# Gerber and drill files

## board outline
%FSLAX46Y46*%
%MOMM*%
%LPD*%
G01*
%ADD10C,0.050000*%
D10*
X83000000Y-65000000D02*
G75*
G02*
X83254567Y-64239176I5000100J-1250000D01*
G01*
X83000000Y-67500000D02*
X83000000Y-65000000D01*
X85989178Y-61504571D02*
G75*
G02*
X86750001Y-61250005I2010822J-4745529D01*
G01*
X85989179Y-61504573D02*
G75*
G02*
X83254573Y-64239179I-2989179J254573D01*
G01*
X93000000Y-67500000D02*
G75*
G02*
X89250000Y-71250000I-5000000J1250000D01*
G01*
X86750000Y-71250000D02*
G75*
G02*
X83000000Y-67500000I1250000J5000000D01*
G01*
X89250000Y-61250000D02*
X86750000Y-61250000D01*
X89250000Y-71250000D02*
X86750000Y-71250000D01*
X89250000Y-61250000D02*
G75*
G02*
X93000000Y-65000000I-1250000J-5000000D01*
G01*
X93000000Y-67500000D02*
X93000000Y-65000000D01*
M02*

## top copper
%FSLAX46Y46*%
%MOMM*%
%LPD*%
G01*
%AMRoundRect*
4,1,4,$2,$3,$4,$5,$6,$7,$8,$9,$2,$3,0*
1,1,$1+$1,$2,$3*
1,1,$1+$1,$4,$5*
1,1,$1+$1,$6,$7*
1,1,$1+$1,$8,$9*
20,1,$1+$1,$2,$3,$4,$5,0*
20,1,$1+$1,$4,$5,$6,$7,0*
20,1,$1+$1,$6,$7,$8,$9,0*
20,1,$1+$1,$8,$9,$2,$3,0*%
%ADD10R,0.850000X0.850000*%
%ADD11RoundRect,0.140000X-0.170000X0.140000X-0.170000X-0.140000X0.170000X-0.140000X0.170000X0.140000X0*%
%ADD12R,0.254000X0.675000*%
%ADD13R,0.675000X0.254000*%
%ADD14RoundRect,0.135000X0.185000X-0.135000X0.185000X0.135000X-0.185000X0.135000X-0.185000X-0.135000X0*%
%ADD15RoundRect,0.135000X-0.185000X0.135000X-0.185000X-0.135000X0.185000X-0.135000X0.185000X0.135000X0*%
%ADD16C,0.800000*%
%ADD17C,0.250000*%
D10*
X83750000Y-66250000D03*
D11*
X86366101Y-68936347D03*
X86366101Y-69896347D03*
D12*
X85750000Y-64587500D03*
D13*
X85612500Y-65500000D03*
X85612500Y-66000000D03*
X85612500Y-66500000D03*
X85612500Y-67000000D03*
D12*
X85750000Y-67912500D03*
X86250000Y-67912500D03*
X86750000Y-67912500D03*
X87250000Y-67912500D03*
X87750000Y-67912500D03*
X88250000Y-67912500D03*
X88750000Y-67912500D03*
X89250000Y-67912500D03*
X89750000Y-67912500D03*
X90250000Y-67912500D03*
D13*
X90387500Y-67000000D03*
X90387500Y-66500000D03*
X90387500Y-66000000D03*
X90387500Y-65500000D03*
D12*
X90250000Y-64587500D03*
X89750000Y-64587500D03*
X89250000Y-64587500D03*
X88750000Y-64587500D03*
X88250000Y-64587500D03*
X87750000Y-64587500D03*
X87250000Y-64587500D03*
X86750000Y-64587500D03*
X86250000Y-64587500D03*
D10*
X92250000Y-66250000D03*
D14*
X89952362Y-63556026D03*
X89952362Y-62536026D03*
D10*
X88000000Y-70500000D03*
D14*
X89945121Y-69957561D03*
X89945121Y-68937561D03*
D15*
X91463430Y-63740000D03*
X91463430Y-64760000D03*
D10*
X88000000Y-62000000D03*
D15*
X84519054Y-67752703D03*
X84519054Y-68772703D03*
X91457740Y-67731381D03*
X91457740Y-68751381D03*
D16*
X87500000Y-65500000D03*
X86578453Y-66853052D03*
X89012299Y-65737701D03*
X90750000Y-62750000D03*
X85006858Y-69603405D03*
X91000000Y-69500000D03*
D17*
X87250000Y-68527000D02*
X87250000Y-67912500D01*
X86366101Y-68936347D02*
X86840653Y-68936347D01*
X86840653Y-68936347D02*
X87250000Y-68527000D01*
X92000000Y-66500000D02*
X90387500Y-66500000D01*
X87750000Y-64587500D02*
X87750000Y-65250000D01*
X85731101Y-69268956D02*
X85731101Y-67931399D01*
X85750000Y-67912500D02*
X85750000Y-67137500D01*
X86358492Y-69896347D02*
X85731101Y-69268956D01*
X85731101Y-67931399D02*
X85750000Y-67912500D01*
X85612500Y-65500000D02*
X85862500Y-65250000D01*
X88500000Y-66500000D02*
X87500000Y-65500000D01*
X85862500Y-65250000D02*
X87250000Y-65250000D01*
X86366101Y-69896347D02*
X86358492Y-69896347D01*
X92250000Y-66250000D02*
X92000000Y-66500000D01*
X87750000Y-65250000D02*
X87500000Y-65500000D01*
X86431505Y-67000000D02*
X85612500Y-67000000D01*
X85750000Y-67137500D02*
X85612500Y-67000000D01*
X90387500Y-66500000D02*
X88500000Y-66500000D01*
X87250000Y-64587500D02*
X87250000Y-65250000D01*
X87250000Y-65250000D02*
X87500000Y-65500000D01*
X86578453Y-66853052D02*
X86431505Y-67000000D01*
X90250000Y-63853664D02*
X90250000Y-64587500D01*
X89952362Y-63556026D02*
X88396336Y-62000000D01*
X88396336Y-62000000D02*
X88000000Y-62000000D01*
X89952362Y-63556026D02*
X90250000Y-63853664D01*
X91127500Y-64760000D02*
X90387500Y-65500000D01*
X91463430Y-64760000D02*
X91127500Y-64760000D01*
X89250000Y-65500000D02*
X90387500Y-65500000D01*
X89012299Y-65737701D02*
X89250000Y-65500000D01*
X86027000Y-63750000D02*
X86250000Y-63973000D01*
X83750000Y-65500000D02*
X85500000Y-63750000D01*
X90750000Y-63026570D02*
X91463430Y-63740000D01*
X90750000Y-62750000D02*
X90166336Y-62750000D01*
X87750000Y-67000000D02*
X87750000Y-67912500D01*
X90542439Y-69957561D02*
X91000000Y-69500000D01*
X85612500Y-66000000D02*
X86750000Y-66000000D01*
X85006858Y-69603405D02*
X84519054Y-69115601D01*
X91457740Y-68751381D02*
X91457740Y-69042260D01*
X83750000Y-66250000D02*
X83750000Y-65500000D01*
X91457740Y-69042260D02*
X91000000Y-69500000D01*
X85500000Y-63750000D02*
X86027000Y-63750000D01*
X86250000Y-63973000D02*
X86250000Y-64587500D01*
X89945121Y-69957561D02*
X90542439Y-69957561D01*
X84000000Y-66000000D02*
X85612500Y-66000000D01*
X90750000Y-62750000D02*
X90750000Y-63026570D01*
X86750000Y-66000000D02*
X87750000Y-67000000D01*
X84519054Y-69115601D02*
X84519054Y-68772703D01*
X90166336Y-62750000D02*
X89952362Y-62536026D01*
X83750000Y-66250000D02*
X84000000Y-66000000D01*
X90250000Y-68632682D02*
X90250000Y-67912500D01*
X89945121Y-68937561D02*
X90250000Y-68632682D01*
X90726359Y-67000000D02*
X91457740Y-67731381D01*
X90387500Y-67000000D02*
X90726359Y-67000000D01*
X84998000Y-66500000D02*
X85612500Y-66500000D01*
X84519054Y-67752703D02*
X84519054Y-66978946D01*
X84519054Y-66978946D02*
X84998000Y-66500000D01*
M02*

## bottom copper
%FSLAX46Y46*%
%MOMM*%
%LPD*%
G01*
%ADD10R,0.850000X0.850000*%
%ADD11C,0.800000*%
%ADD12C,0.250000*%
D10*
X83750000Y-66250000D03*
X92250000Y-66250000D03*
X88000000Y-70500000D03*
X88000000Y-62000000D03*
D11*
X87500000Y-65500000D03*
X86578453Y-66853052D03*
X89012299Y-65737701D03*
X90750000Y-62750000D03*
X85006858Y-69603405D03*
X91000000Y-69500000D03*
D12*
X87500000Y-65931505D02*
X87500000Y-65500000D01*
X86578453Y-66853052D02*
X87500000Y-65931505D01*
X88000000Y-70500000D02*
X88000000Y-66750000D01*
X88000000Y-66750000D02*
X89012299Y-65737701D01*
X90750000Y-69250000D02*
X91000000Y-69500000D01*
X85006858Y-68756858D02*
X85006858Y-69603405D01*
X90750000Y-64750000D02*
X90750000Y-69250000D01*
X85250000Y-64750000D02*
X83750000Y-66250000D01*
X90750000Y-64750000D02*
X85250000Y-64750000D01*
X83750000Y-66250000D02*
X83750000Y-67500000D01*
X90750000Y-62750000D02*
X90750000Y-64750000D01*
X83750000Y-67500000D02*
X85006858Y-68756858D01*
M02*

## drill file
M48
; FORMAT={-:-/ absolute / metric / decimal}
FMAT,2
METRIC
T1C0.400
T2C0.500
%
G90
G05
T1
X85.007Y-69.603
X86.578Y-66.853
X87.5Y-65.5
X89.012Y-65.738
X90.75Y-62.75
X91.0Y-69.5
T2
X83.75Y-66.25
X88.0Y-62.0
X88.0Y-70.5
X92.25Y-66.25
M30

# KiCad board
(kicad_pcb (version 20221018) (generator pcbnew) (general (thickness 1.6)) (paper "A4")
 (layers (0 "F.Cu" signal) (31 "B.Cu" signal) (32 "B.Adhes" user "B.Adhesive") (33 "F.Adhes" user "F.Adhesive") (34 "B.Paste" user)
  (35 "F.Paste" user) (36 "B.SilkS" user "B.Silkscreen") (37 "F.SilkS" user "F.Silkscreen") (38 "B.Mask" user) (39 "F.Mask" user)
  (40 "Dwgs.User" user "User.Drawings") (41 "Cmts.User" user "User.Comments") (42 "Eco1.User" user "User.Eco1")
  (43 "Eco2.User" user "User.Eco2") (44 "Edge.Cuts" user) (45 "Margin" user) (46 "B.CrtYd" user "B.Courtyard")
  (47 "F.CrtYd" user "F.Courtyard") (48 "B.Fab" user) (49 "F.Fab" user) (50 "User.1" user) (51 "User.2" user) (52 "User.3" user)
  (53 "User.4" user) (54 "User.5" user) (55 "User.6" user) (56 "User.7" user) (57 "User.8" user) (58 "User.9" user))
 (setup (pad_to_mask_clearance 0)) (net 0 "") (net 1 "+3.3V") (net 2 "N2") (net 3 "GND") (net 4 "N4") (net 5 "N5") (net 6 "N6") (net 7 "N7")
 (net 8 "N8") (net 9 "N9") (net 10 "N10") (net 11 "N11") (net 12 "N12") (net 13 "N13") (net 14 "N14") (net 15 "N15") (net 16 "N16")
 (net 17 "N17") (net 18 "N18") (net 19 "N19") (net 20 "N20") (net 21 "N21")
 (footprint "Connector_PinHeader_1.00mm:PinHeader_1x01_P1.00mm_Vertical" (layer "F.Cu") (at 83.75 66.25)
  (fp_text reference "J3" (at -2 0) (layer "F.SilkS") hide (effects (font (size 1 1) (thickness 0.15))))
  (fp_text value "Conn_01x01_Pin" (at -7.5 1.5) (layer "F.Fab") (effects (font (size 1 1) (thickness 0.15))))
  (pad "1" thru_hole rect (at 0 0) (size 0.85 0.85) (drill 0.5) (layers "*.Cu" "*.Mask") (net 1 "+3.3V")))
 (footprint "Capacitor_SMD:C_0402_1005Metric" (layer "F.Cu") (at 86.366101 69.416347 -90)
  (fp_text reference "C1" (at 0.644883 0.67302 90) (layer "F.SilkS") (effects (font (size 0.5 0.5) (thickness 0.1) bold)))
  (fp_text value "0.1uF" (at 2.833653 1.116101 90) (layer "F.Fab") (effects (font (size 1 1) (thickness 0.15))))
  (pad "1" smd roundrect (at -0.48 0 270) (size 0.56 0.62) (layers "F.Cu" "F.Paste" "F.Mask") (roundrect_rratio 0.25) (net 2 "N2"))
  (pad "2" smd roundrect (at 0.48 0 270) (size 0.56 0.62) (layers "F.Cu" "F.Paste" "F.Mask") (roundrect_rratio 0.25) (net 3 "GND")))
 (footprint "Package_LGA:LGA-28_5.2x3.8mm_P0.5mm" (layer "F.Cu") (at 88 66.25)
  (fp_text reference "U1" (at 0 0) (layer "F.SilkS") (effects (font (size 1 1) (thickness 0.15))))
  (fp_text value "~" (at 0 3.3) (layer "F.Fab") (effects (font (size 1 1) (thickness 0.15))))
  (pad "1" smd rect (at -2.25 -1.6625) (size 0.254 0.675) (layers "F.Cu" "F.Paste" "F.Mask") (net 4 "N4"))
  (pad "2" smd rect (at -2.3875 -0.75 90) (size 0.254 0.675) (layers "F.Cu" "F.Paste" "F.Mask") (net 3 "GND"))
  (pad "3" smd rect (at -2.3875 -0.25 90) (size 0.254 0.675) (layers "F.Cu" "F.Paste" "F.Mask") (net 1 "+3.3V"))
  (pad "4" smd rect (at -2.3875 0.25 90) (size 0.254 0.675) (layers "F.Cu" "F.Paste" "F.Mask") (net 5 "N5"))
  (pad "5" smd rect (at -2.3875 0.75 90) (size 0.254 0.675) (layers "F.Cu" "F.Paste" "F.Mask") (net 3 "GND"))
  (pad "6" smd rect (at -2.25 1.6625) (size 0.254 0.675) (layers "F.Cu" "F.Paste" "F.Mask") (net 3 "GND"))
  (pad "7" smd rect (at -1.75 1.6625) (size 0.254 0.675) (layers "F.Cu" "F.Paste" "F.Mask") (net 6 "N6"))
  (pad "8" smd rect (at -1.25 1.6625) (size 0.254 0.675) (layers "F.Cu" "F.Paste" "F.Mask") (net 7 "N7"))
  (pad "9" smd rect (at -0.75 1.6625) (size 0.254 0.675) (layers "F.Cu" "F.Paste" "F.Mask") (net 2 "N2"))
  (pad "10" smd rect (at -0.25 1.6625) (size 0.254 0.675) (layers "F.Cu" "F.Paste" "F.Mask") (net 1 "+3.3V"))
  (pad "11" smd rect (at 0.25 1.6625) (size 0.254 0.675) (layers "F.Cu" "F.Paste" "F.Mask") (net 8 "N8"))
  (pad "12" smd rect (at 0.75 1.6625) (size 0.254 0.675) (layers "F.Cu" "F.Paste" "F.Mask") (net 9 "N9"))
  (pad "13" smd rect (at 1.25 1.6625) (size 0.254 0.675) (layers "F.Cu" "F.Paste" "F.Mask") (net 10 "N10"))
  (pad "14" smd rect (at 1.75 1.6625) (size 0.254 0.675) (layers "F.Cu" "F.Paste" "F.Mask") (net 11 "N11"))
  (pad "15" smd rect (at 2.25 1.6625) (size 0.254 0.675) (layers "F.Cu" "F.Paste" "F.Mask") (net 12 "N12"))
  (pad "16" smd rect (at 2.3875 0.75 90) (size 0.254 0.675) (layers "F.Cu" "F.Paste" "F.Mask") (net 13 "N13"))
  (pad "17" smd rect (at 2.3875 0.25 90) (size 0.254 0.675) (layers "F.Cu" "F.Paste" "F.Mask") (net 3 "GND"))
  (pad "18" smd rect (at 2.3875 -0.25 90) (size 0.254 0.675) (layers "F.Cu" "F.Paste" "F.Mask") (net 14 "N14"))
  (pad "19" smd rect (at 2.3875 -0.75 90) (size 0.254 0.675) (layers "F.Cu" "F.Paste" "F.Mask") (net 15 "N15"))
  (pad "20" smd rect (at 2.25 -1.6625) (size 0.254 0.675) (layers "F.Cu" "F.Paste" "F.Mask") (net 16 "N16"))
  (pad "21" smd rect (at 1.75 -1.6625) (size 0.254 0.675) (layers "F.Cu" "F.Paste" "F.Mask") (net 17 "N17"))
  (pad "22" smd rect (at 1.25 -1.6625) (size 0.254 0.675) (layers "F.Cu" "F.Paste" "F.Mask") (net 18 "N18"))
  (pad "23" smd rect (at 0.75 -1.6625) (size 0.254 0.675) (layers "F.Cu" "F.Paste" "F.Mask") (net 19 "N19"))
  (pad "24" smd rect (at 0.25 -1.6625) (size 0.254 0.675) (layers "F.Cu" "F.Paste" "F.Mask") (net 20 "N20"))
  (pad "25" smd rect (at -0.25 -1.6625) (size 0.254 0.675) (layers "F.Cu" "F.Paste" "F.Mask") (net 3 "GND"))
  (pad "26" smd rect (at -0.75 -1.6625) (size 0.254 0.675) (layers "F.Cu" "F.Paste" "F.Mask") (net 3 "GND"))
  (pad "27" smd rect (at -1.25 -1.6625) (size 0.254 0.675) (layers "F.Cu" "F.Paste" "F.Mask") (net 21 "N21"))
  (pad "28" smd rect (at -1.75 -1.6625) (size 0.254 0.675) (layers "F.Cu" "F.Paste" "F.Mask") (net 1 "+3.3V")))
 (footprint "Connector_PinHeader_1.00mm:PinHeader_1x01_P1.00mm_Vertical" (layer "F.Cu") (at 92.25 66.25)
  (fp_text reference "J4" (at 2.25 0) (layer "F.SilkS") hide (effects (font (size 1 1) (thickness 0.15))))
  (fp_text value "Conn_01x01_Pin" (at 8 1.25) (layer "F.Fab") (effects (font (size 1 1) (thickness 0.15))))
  (pad "1" thru_hole rect (at 0 0) (size 0.85 0.85) (drill 0.5) (layers "*.Cu" "*.Mask") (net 3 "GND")))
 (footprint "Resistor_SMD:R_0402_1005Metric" (layer "F.Cu") (at 89.952362 63.046026 90)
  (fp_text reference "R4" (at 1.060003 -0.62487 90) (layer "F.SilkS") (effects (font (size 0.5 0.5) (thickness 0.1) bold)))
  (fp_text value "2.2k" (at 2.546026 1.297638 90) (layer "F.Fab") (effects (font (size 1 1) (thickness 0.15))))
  (pad "1" smd roundrect (at -0.51 0 90) (size 0.54 0.64) (layers "F.Cu" "F.Paste" "F.Mask") (roundrect_rratio 0.25) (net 16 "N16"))
  (pad "2" smd roundrect (at 0.51 0 90) (size 0.54 0.64) (layers "F.Cu" "F.Paste" "F.Mask") (roundrect_rratio 0.25) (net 1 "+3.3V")))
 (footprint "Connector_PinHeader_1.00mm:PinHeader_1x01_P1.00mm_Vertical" (layer "F.Cu") (at 88 70.5)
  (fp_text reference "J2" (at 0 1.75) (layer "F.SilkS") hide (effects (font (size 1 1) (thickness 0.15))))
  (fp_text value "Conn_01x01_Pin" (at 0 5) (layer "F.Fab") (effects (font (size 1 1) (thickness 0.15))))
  (pad "1" thru_hole rect (at 0 0) (size 0.85 0.85) (drill 0.5) (layers "*.Cu" "*.Mask") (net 15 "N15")))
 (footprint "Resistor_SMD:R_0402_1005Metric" (layer "F.Cu") (at 89.945121 69.447561 90)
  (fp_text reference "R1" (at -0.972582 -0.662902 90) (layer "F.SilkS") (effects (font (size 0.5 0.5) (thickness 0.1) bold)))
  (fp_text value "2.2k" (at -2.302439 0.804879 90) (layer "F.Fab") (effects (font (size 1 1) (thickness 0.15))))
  (pad "1" smd roundrect (at -0.51 0 90) (size 0.54 0.64) (layers "F.Cu" "F.Paste" "F.Mask") (roundrect_rratio 0.25) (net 1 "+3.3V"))
  (pad "2" smd roundrect (at 0.51 0 90) (size 0.54 0.64) (layers "F.Cu" "F.Paste" "F.Mask") (roundrect_rratio 0.25) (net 12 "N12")))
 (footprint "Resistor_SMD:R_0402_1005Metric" (layer "F.Cu") (at 91.46343 64.25 -90)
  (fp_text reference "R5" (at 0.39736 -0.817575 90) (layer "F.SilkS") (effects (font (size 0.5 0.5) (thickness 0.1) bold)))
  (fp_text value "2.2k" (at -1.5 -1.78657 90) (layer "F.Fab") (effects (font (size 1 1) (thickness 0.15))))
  (pad "1" smd roundrect (at -0.51 0 270) (size 0.54 0.64) (layers "F.Cu" "F.Paste" "F.Mask") (roundrect_rratio 0.25) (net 1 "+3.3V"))
  (pad "2" smd roundrect (at 0.51 0 270) (size 0.54 0.64) (layers "F.Cu" "F.Paste" "F.Mask") (roundrect_rratio 0.25) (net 15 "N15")))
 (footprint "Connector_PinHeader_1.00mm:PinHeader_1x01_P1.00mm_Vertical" (layer "F.Cu") (at 88 62)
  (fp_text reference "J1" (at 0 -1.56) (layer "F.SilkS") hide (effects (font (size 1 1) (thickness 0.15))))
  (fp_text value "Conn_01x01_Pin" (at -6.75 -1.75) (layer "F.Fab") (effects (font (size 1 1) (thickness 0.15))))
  (pad "1" thru_hole rect (at 0 0) (size 0.85 0.85) (drill 0.5) (layers "*.Cu" "*.Mask") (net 16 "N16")))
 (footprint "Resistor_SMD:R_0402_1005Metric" (layer "F.Cu") (at 84.519054 68.262703 -90)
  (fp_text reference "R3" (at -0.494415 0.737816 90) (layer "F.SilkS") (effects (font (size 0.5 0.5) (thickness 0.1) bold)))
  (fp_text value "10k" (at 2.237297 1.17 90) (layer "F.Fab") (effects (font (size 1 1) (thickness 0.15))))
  (pad "1" smd roundrect (at -0.51 0 270) (size 0.54 0.64) (layers "F.Cu" "F.Paste" "F.Mask") (roundrect_rratio 0.25) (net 5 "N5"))
  (pad "2" smd roundrect (at 0.51 0 270) (size 0.54 0.64) (layers "F.Cu" "F.Paste" "F.Mask") (roundrect_rratio 0.25) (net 1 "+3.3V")))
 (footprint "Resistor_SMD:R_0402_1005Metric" (layer "F.Cu") (at 91.45774 68.241381 -90)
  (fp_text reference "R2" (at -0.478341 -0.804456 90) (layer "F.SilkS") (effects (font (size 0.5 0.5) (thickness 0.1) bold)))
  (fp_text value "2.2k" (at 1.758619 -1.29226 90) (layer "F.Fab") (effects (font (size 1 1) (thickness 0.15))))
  (pad "1" smd roundrect (at -0.51 0 270) (size 0.54 0.64) (layers "F.Cu" "F.Paste" "F.Mask") (roundrect_rratio 0.25) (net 13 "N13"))
  (pad "2" smd roundrect (at 0.51 0 270) (size 0.54 0.64) (layers "F.Cu" "F.Paste" "F.Mask") (roundrect_rratio 0.25) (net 1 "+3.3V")))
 (gr_arc (start 83 65) (mid 83.112459 64.614628) (end 83.254571 64.239178) (stroke (width 0.05) (type default)) (layer "Edge.Cuts"))
 (gr_line (start 83 67.5) (end 83 65) (stroke (width 0.05) (type default)) (layer "Edge.Cuts"))
 (gr_arc (start 85.989178 61.504571) (mid 86.364628 61.362459) (end 86.75 61.25) (stroke (width 0.05) (type default)) (layer "Edge.Cuts"))
 (gr_arc (start 85.989179 61.504573) (mid 85.12132 63.37132) (end 83.254573 64.239179) (stroke (width 0.05) (type default))
  (layer "Edge.Cuts"))
 (gr_arc (start 93 67.5) (mid 91.644345 69.894345) (end 89.25 71.25) (stroke (width 0.05) (type default)) (layer "Edge.Cuts"))
 (gr_arc (start 86.75 71.25) (mid 84.355655 69.894345) (end 83 67.5) (stroke (width 0.05) (type default)) (layer "Edge.Cuts"))
 (gr_line (start 89.25 61.25) (end 86.75 61.25) (stroke (width 0.05) (type default)) (layer "Edge.Cuts"))
 (gr_line (start 89.25 71.25) (end 86.75 71.25) (stroke (width 0.05) (type default)) (layer "Edge.Cuts"))
 (gr_arc (start 89.25 61.25) (mid 91.644345 62.605655) (end 93 65) (stroke (width 0.05) (type default)) (layer "Edge.Cuts"))
 (gr_line (start 93 67.5) (end 93 65) (stroke (width 0.05) (type default)) (layer "Edge.Cuts"))
 (segment (start 87.25 68.527) (end 87.25 67.9125) (width 0.25) (layer "F.Cu") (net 2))
 (segment (start 86.366101 68.936347) (end 86.840653 68.936347) (width 0.25) (layer "F.Cu") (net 2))
 (segment (start 86.840653 68.936347) (end 87.25 68.527) (width 0.25) (layer "F.Cu") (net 2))
 (segment (start 92 66.5) (end 90.3875 66.5) (width 0.25) (layer "F.Cu") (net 3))
 (segment (start 87.75 64.5875) (end 87.75 65.25) (width 0.25) (layer "F.Cu") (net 3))
 (segment (start 85.731101 69.268956) (end 85.731101 67.931399) (width 0.25) (layer "F.Cu") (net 3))
 (segment (start 85.75 67.9125) (end 85.75 67.1375) (width 0.25) (layer "F.Cu") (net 3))
 (segment (start 86.358492 69.896347) (end 85.731101 69.268956) (width 0.25) (layer "F.Cu") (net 3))
 (segment (start 85.731101 67.931399) (end 85.75 67.9125) (width 0.25) (layer "F.Cu") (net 3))
 (segment (start 85.6125 65.5) (end 85.8625 65.25) (width 0.25) (layer "F.Cu") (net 3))
 (segment (start 88.5 66.5) (end 87.5 65.5) (width 0.25) (layer "F.Cu") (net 3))
 (segment (start 85.8625 65.25) (end 87.25 65.25) (width 0.25) (layer "F.Cu") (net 3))
 (segment (start 86.366101 69.896347) (end 86.358492 69.896347) (width 0.25) (layer "F.Cu") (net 3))
 (segment (start 92.25 66.25) (end 92 66.5) (width 0.25) (layer "F.Cu") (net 3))
 (segment (start 87.75 65.25) (end 87.5 65.5) (width 0.25) (layer "F.Cu") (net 3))
 (segment (start 86.431505 67) (end 85.6125 67) (width 0.25) (layer "F.Cu") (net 3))
 (segment (start 85.75 67.1375) (end 85.6125 67) (width 0.25) (layer "F.Cu") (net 3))
 (segment (start 90.3875 66.5) (end 88.5 66.5) (width 0.25) (layer "F.Cu") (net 3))
 (segment (start 87.25 64.5875) (end 87.25 65.25) (width 0.25) (layer "F.Cu") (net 3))
 (segment (start 87.25 65.25) (end 87.5 65.5) (width 0.25) (layer "F.Cu") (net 3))
 (segment (start 86.578453 66.853052) (end 86.431505 67) (width 0.25) (layer "F.Cu") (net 3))
 (via (at 87.5 65.5) (size 0.8) (drill 0.4) (layers "F.Cu" "B.Cu") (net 3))
 (via (at 86.578453 66.853052) (size 0.8) (drill 0.4) (layers "F.Cu" "B.Cu") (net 3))
 (segment (start 87.5 65.931505) (end 87.5 65.5) (width 0.25) (layer "B.Cu") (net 3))
 (segment (start 86.578453 66.853052) (end 87.5 65.931505) (width 0.25) (layer "B.Cu") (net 3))
 (segment (start 90.25 63.853664) (end 90.25 64.5875) (width 0.25) (layer "F.Cu") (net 16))
 (segment (start 89.952362 63.556026) (end 88.396336 62) (width 0.25) (layer "F.Cu") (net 16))
 (segment (start 88.396336 62) (end 88 62) (width 0.25) (layer "F.Cu") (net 16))
 (segment (start 89.952362 63.556026) (end 90.25 63.853664) (width 0.25) (layer "F.Cu") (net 16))
 (segment (start 91.1275 64.76) (end 90.3875 65.5) (width 0.25) (layer "F.Cu") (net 15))
 (segment (start 91.46343 64.76) (end 91.1275 64.76) (width 0.25) (layer "F.Cu") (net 15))
 (segment (start 89.25 65.5) (end 90.3875 65.5) (width 0.25) (layer "F.Cu") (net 15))
 (segment (start 89.012299 65.737701) (end 89.25 65.5) (width 0.25) (layer "F.Cu") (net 15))
 (via (at 89.012299 65.737701) (size 0.8) (drill 0.4) (layers "F.Cu" "B.Cu") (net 15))
 (segment (start 88 70.5) (end 88 66.75) (width 0.25) (layer "B.Cu") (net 15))
 (segment (start 88 66.75) (end 89.012299 65.737701) (width 0.25) (layer "B.Cu") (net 15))
 (segment (start 86.027 63.75) (end 86.25 63.973) (width 0.25) (layer "F.Cu") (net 1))
 (segment (start 83.75 65.5) (end 85.5 63.75) (width 0.25) (layer "F.Cu") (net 1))
 (segment (start 90.75 63.02657) (end 91.46343 63.74) (width 0.25) (layer "F.Cu") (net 1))
 (segment (start 90.75 62.75) (end 90.166336 62.75) (width 0.25) (layer "F.Cu") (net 1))
 (segment (start 87.75 67) (end 87.75 67.9125) (width 0.25) (layer "F.Cu") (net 1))
 (segment (start 90.542439 69.957561) (end 91 69.5) (width 0.25) (layer "F.Cu") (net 1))
 (segment (start 85.6125 66) (end 86.75 66) (width 0.25) (layer "F.Cu") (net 1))
 (segment (start 85.006858 69.603405) (end 84.519054 69.115601) (width 0.25) (layer "F.Cu") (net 1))
 (segment (start 91.45774 68.751381) (end 91.45774 69.04226) (width 0.25) (layer "F.Cu") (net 1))
 (segment (start 83.75 66.25) (end 83.75 65.5) (width 0.25) (layer "F.Cu") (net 1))
 (segment (start 91.45774 69.04226) (end 91 69.5) (width 0.25) (layer "F.Cu") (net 1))
 (segment (start 85.5 63.75) (end 86.027 63.75) (width 0.25) (layer "F.Cu") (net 1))
 (segment (start 86.25 63.973) (end 86.25 64.5875) (width 0.25) (layer "F.Cu") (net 1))
 (segment (start 89.945121 69.957561) (end 90.542439 69.957561) (width 0.25) (layer "F.Cu") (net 1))
 (segment (start 84 66) (end 85.6125 66) (width 0.25) (layer "F.Cu") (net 1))
 (segment (start 90.75 62.75) (end 90.75 63.02657) (width 0.25) (layer "F.Cu") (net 1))
 (segment (start 86.75 66) (end 87.75 67) (width 0.25) (layer "F.Cu") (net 1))
 (segment (start 84.519054 69.115601) (end 84.519054 68.772703) (width 0.25) (layer "F.Cu") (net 1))
 (segment (start 90.166336 62.75) (end 89.952362 62.536026) (width 0.25) (layer "F.Cu") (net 1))
 (segment (start 83.75 66.25) (end 84 66) (width 0.25) (layer "F.Cu") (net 1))
 (via (at 90.75 62.75) (size 0.8) (drill 0.4) (layers "F.Cu" "B.Cu") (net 1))
 (via (at 85.006858 69.603405) (size 0.8) (drill 0.4) (layers "F.Cu" "B.Cu") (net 1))
 (via (at 91 69.5) (size 0.8) (drill 0.4) (layers "F.Cu" "B.Cu") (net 1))
 (segment (start 90.75 69.25) (end 91 69.5) (width 0.25) (layer "B.Cu") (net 1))
 (segment (start 85.006858 68.756858) (end 85.006858 69.603405) (width 0.25) (layer "B.Cu") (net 1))
 (segment (start 90.75 64.75) (end 90.75 69.25) (width 0.25) (layer "B.Cu") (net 1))
 (segment (start 85.25 64.75) (end 83.75 66.25) (width 0.25) (layer "B.Cu") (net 1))
 (segment (start 90.75 64.75) (end 85.25 64.75) (width 0.25) (layer "B.Cu") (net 1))
 (segment (start 83.75 66.25) (end 83.75 67.5) (width 0.25) (layer "B.Cu") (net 1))
 (segment (start 90.75 62.75) (end 90.75 64.75) (width 0.25) (layer "B.Cu") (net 1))
 (segment (start 83.75 67.5) (end 85.006858 68.756858) (width 0.25) (layer "B.Cu") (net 1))
 (segment (start 90.25 68.632682) (end 90.25 67.9125) (width 0.25) (layer "F.Cu") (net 12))
 (segment (start 89.945121 68.937561) (end 90.25 68.632682) (width 0.25) (layer "F.Cu") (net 12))
 (segment (start 90.726359 67) (end 91.45774 67.731381) (width 0.25) (layer "F.Cu") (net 13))
 (segment (start 90.3875 67) (end 90.726359 67) (width 0.25) (layer "F.Cu") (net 13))
 (segment (start 84.998 66.5) (end 85.6125 66.5) (width 0.25) (layer "F.Cu") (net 5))
 (segment (start 84.519054 67.752703) (end 84.519054 66.978946) (width 0.25) (layer "F.Cu") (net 5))
 (segment (start 84.519054 66.978946) (end 84.998 66.5) (width 0.25) (layer "F.Cu") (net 5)))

